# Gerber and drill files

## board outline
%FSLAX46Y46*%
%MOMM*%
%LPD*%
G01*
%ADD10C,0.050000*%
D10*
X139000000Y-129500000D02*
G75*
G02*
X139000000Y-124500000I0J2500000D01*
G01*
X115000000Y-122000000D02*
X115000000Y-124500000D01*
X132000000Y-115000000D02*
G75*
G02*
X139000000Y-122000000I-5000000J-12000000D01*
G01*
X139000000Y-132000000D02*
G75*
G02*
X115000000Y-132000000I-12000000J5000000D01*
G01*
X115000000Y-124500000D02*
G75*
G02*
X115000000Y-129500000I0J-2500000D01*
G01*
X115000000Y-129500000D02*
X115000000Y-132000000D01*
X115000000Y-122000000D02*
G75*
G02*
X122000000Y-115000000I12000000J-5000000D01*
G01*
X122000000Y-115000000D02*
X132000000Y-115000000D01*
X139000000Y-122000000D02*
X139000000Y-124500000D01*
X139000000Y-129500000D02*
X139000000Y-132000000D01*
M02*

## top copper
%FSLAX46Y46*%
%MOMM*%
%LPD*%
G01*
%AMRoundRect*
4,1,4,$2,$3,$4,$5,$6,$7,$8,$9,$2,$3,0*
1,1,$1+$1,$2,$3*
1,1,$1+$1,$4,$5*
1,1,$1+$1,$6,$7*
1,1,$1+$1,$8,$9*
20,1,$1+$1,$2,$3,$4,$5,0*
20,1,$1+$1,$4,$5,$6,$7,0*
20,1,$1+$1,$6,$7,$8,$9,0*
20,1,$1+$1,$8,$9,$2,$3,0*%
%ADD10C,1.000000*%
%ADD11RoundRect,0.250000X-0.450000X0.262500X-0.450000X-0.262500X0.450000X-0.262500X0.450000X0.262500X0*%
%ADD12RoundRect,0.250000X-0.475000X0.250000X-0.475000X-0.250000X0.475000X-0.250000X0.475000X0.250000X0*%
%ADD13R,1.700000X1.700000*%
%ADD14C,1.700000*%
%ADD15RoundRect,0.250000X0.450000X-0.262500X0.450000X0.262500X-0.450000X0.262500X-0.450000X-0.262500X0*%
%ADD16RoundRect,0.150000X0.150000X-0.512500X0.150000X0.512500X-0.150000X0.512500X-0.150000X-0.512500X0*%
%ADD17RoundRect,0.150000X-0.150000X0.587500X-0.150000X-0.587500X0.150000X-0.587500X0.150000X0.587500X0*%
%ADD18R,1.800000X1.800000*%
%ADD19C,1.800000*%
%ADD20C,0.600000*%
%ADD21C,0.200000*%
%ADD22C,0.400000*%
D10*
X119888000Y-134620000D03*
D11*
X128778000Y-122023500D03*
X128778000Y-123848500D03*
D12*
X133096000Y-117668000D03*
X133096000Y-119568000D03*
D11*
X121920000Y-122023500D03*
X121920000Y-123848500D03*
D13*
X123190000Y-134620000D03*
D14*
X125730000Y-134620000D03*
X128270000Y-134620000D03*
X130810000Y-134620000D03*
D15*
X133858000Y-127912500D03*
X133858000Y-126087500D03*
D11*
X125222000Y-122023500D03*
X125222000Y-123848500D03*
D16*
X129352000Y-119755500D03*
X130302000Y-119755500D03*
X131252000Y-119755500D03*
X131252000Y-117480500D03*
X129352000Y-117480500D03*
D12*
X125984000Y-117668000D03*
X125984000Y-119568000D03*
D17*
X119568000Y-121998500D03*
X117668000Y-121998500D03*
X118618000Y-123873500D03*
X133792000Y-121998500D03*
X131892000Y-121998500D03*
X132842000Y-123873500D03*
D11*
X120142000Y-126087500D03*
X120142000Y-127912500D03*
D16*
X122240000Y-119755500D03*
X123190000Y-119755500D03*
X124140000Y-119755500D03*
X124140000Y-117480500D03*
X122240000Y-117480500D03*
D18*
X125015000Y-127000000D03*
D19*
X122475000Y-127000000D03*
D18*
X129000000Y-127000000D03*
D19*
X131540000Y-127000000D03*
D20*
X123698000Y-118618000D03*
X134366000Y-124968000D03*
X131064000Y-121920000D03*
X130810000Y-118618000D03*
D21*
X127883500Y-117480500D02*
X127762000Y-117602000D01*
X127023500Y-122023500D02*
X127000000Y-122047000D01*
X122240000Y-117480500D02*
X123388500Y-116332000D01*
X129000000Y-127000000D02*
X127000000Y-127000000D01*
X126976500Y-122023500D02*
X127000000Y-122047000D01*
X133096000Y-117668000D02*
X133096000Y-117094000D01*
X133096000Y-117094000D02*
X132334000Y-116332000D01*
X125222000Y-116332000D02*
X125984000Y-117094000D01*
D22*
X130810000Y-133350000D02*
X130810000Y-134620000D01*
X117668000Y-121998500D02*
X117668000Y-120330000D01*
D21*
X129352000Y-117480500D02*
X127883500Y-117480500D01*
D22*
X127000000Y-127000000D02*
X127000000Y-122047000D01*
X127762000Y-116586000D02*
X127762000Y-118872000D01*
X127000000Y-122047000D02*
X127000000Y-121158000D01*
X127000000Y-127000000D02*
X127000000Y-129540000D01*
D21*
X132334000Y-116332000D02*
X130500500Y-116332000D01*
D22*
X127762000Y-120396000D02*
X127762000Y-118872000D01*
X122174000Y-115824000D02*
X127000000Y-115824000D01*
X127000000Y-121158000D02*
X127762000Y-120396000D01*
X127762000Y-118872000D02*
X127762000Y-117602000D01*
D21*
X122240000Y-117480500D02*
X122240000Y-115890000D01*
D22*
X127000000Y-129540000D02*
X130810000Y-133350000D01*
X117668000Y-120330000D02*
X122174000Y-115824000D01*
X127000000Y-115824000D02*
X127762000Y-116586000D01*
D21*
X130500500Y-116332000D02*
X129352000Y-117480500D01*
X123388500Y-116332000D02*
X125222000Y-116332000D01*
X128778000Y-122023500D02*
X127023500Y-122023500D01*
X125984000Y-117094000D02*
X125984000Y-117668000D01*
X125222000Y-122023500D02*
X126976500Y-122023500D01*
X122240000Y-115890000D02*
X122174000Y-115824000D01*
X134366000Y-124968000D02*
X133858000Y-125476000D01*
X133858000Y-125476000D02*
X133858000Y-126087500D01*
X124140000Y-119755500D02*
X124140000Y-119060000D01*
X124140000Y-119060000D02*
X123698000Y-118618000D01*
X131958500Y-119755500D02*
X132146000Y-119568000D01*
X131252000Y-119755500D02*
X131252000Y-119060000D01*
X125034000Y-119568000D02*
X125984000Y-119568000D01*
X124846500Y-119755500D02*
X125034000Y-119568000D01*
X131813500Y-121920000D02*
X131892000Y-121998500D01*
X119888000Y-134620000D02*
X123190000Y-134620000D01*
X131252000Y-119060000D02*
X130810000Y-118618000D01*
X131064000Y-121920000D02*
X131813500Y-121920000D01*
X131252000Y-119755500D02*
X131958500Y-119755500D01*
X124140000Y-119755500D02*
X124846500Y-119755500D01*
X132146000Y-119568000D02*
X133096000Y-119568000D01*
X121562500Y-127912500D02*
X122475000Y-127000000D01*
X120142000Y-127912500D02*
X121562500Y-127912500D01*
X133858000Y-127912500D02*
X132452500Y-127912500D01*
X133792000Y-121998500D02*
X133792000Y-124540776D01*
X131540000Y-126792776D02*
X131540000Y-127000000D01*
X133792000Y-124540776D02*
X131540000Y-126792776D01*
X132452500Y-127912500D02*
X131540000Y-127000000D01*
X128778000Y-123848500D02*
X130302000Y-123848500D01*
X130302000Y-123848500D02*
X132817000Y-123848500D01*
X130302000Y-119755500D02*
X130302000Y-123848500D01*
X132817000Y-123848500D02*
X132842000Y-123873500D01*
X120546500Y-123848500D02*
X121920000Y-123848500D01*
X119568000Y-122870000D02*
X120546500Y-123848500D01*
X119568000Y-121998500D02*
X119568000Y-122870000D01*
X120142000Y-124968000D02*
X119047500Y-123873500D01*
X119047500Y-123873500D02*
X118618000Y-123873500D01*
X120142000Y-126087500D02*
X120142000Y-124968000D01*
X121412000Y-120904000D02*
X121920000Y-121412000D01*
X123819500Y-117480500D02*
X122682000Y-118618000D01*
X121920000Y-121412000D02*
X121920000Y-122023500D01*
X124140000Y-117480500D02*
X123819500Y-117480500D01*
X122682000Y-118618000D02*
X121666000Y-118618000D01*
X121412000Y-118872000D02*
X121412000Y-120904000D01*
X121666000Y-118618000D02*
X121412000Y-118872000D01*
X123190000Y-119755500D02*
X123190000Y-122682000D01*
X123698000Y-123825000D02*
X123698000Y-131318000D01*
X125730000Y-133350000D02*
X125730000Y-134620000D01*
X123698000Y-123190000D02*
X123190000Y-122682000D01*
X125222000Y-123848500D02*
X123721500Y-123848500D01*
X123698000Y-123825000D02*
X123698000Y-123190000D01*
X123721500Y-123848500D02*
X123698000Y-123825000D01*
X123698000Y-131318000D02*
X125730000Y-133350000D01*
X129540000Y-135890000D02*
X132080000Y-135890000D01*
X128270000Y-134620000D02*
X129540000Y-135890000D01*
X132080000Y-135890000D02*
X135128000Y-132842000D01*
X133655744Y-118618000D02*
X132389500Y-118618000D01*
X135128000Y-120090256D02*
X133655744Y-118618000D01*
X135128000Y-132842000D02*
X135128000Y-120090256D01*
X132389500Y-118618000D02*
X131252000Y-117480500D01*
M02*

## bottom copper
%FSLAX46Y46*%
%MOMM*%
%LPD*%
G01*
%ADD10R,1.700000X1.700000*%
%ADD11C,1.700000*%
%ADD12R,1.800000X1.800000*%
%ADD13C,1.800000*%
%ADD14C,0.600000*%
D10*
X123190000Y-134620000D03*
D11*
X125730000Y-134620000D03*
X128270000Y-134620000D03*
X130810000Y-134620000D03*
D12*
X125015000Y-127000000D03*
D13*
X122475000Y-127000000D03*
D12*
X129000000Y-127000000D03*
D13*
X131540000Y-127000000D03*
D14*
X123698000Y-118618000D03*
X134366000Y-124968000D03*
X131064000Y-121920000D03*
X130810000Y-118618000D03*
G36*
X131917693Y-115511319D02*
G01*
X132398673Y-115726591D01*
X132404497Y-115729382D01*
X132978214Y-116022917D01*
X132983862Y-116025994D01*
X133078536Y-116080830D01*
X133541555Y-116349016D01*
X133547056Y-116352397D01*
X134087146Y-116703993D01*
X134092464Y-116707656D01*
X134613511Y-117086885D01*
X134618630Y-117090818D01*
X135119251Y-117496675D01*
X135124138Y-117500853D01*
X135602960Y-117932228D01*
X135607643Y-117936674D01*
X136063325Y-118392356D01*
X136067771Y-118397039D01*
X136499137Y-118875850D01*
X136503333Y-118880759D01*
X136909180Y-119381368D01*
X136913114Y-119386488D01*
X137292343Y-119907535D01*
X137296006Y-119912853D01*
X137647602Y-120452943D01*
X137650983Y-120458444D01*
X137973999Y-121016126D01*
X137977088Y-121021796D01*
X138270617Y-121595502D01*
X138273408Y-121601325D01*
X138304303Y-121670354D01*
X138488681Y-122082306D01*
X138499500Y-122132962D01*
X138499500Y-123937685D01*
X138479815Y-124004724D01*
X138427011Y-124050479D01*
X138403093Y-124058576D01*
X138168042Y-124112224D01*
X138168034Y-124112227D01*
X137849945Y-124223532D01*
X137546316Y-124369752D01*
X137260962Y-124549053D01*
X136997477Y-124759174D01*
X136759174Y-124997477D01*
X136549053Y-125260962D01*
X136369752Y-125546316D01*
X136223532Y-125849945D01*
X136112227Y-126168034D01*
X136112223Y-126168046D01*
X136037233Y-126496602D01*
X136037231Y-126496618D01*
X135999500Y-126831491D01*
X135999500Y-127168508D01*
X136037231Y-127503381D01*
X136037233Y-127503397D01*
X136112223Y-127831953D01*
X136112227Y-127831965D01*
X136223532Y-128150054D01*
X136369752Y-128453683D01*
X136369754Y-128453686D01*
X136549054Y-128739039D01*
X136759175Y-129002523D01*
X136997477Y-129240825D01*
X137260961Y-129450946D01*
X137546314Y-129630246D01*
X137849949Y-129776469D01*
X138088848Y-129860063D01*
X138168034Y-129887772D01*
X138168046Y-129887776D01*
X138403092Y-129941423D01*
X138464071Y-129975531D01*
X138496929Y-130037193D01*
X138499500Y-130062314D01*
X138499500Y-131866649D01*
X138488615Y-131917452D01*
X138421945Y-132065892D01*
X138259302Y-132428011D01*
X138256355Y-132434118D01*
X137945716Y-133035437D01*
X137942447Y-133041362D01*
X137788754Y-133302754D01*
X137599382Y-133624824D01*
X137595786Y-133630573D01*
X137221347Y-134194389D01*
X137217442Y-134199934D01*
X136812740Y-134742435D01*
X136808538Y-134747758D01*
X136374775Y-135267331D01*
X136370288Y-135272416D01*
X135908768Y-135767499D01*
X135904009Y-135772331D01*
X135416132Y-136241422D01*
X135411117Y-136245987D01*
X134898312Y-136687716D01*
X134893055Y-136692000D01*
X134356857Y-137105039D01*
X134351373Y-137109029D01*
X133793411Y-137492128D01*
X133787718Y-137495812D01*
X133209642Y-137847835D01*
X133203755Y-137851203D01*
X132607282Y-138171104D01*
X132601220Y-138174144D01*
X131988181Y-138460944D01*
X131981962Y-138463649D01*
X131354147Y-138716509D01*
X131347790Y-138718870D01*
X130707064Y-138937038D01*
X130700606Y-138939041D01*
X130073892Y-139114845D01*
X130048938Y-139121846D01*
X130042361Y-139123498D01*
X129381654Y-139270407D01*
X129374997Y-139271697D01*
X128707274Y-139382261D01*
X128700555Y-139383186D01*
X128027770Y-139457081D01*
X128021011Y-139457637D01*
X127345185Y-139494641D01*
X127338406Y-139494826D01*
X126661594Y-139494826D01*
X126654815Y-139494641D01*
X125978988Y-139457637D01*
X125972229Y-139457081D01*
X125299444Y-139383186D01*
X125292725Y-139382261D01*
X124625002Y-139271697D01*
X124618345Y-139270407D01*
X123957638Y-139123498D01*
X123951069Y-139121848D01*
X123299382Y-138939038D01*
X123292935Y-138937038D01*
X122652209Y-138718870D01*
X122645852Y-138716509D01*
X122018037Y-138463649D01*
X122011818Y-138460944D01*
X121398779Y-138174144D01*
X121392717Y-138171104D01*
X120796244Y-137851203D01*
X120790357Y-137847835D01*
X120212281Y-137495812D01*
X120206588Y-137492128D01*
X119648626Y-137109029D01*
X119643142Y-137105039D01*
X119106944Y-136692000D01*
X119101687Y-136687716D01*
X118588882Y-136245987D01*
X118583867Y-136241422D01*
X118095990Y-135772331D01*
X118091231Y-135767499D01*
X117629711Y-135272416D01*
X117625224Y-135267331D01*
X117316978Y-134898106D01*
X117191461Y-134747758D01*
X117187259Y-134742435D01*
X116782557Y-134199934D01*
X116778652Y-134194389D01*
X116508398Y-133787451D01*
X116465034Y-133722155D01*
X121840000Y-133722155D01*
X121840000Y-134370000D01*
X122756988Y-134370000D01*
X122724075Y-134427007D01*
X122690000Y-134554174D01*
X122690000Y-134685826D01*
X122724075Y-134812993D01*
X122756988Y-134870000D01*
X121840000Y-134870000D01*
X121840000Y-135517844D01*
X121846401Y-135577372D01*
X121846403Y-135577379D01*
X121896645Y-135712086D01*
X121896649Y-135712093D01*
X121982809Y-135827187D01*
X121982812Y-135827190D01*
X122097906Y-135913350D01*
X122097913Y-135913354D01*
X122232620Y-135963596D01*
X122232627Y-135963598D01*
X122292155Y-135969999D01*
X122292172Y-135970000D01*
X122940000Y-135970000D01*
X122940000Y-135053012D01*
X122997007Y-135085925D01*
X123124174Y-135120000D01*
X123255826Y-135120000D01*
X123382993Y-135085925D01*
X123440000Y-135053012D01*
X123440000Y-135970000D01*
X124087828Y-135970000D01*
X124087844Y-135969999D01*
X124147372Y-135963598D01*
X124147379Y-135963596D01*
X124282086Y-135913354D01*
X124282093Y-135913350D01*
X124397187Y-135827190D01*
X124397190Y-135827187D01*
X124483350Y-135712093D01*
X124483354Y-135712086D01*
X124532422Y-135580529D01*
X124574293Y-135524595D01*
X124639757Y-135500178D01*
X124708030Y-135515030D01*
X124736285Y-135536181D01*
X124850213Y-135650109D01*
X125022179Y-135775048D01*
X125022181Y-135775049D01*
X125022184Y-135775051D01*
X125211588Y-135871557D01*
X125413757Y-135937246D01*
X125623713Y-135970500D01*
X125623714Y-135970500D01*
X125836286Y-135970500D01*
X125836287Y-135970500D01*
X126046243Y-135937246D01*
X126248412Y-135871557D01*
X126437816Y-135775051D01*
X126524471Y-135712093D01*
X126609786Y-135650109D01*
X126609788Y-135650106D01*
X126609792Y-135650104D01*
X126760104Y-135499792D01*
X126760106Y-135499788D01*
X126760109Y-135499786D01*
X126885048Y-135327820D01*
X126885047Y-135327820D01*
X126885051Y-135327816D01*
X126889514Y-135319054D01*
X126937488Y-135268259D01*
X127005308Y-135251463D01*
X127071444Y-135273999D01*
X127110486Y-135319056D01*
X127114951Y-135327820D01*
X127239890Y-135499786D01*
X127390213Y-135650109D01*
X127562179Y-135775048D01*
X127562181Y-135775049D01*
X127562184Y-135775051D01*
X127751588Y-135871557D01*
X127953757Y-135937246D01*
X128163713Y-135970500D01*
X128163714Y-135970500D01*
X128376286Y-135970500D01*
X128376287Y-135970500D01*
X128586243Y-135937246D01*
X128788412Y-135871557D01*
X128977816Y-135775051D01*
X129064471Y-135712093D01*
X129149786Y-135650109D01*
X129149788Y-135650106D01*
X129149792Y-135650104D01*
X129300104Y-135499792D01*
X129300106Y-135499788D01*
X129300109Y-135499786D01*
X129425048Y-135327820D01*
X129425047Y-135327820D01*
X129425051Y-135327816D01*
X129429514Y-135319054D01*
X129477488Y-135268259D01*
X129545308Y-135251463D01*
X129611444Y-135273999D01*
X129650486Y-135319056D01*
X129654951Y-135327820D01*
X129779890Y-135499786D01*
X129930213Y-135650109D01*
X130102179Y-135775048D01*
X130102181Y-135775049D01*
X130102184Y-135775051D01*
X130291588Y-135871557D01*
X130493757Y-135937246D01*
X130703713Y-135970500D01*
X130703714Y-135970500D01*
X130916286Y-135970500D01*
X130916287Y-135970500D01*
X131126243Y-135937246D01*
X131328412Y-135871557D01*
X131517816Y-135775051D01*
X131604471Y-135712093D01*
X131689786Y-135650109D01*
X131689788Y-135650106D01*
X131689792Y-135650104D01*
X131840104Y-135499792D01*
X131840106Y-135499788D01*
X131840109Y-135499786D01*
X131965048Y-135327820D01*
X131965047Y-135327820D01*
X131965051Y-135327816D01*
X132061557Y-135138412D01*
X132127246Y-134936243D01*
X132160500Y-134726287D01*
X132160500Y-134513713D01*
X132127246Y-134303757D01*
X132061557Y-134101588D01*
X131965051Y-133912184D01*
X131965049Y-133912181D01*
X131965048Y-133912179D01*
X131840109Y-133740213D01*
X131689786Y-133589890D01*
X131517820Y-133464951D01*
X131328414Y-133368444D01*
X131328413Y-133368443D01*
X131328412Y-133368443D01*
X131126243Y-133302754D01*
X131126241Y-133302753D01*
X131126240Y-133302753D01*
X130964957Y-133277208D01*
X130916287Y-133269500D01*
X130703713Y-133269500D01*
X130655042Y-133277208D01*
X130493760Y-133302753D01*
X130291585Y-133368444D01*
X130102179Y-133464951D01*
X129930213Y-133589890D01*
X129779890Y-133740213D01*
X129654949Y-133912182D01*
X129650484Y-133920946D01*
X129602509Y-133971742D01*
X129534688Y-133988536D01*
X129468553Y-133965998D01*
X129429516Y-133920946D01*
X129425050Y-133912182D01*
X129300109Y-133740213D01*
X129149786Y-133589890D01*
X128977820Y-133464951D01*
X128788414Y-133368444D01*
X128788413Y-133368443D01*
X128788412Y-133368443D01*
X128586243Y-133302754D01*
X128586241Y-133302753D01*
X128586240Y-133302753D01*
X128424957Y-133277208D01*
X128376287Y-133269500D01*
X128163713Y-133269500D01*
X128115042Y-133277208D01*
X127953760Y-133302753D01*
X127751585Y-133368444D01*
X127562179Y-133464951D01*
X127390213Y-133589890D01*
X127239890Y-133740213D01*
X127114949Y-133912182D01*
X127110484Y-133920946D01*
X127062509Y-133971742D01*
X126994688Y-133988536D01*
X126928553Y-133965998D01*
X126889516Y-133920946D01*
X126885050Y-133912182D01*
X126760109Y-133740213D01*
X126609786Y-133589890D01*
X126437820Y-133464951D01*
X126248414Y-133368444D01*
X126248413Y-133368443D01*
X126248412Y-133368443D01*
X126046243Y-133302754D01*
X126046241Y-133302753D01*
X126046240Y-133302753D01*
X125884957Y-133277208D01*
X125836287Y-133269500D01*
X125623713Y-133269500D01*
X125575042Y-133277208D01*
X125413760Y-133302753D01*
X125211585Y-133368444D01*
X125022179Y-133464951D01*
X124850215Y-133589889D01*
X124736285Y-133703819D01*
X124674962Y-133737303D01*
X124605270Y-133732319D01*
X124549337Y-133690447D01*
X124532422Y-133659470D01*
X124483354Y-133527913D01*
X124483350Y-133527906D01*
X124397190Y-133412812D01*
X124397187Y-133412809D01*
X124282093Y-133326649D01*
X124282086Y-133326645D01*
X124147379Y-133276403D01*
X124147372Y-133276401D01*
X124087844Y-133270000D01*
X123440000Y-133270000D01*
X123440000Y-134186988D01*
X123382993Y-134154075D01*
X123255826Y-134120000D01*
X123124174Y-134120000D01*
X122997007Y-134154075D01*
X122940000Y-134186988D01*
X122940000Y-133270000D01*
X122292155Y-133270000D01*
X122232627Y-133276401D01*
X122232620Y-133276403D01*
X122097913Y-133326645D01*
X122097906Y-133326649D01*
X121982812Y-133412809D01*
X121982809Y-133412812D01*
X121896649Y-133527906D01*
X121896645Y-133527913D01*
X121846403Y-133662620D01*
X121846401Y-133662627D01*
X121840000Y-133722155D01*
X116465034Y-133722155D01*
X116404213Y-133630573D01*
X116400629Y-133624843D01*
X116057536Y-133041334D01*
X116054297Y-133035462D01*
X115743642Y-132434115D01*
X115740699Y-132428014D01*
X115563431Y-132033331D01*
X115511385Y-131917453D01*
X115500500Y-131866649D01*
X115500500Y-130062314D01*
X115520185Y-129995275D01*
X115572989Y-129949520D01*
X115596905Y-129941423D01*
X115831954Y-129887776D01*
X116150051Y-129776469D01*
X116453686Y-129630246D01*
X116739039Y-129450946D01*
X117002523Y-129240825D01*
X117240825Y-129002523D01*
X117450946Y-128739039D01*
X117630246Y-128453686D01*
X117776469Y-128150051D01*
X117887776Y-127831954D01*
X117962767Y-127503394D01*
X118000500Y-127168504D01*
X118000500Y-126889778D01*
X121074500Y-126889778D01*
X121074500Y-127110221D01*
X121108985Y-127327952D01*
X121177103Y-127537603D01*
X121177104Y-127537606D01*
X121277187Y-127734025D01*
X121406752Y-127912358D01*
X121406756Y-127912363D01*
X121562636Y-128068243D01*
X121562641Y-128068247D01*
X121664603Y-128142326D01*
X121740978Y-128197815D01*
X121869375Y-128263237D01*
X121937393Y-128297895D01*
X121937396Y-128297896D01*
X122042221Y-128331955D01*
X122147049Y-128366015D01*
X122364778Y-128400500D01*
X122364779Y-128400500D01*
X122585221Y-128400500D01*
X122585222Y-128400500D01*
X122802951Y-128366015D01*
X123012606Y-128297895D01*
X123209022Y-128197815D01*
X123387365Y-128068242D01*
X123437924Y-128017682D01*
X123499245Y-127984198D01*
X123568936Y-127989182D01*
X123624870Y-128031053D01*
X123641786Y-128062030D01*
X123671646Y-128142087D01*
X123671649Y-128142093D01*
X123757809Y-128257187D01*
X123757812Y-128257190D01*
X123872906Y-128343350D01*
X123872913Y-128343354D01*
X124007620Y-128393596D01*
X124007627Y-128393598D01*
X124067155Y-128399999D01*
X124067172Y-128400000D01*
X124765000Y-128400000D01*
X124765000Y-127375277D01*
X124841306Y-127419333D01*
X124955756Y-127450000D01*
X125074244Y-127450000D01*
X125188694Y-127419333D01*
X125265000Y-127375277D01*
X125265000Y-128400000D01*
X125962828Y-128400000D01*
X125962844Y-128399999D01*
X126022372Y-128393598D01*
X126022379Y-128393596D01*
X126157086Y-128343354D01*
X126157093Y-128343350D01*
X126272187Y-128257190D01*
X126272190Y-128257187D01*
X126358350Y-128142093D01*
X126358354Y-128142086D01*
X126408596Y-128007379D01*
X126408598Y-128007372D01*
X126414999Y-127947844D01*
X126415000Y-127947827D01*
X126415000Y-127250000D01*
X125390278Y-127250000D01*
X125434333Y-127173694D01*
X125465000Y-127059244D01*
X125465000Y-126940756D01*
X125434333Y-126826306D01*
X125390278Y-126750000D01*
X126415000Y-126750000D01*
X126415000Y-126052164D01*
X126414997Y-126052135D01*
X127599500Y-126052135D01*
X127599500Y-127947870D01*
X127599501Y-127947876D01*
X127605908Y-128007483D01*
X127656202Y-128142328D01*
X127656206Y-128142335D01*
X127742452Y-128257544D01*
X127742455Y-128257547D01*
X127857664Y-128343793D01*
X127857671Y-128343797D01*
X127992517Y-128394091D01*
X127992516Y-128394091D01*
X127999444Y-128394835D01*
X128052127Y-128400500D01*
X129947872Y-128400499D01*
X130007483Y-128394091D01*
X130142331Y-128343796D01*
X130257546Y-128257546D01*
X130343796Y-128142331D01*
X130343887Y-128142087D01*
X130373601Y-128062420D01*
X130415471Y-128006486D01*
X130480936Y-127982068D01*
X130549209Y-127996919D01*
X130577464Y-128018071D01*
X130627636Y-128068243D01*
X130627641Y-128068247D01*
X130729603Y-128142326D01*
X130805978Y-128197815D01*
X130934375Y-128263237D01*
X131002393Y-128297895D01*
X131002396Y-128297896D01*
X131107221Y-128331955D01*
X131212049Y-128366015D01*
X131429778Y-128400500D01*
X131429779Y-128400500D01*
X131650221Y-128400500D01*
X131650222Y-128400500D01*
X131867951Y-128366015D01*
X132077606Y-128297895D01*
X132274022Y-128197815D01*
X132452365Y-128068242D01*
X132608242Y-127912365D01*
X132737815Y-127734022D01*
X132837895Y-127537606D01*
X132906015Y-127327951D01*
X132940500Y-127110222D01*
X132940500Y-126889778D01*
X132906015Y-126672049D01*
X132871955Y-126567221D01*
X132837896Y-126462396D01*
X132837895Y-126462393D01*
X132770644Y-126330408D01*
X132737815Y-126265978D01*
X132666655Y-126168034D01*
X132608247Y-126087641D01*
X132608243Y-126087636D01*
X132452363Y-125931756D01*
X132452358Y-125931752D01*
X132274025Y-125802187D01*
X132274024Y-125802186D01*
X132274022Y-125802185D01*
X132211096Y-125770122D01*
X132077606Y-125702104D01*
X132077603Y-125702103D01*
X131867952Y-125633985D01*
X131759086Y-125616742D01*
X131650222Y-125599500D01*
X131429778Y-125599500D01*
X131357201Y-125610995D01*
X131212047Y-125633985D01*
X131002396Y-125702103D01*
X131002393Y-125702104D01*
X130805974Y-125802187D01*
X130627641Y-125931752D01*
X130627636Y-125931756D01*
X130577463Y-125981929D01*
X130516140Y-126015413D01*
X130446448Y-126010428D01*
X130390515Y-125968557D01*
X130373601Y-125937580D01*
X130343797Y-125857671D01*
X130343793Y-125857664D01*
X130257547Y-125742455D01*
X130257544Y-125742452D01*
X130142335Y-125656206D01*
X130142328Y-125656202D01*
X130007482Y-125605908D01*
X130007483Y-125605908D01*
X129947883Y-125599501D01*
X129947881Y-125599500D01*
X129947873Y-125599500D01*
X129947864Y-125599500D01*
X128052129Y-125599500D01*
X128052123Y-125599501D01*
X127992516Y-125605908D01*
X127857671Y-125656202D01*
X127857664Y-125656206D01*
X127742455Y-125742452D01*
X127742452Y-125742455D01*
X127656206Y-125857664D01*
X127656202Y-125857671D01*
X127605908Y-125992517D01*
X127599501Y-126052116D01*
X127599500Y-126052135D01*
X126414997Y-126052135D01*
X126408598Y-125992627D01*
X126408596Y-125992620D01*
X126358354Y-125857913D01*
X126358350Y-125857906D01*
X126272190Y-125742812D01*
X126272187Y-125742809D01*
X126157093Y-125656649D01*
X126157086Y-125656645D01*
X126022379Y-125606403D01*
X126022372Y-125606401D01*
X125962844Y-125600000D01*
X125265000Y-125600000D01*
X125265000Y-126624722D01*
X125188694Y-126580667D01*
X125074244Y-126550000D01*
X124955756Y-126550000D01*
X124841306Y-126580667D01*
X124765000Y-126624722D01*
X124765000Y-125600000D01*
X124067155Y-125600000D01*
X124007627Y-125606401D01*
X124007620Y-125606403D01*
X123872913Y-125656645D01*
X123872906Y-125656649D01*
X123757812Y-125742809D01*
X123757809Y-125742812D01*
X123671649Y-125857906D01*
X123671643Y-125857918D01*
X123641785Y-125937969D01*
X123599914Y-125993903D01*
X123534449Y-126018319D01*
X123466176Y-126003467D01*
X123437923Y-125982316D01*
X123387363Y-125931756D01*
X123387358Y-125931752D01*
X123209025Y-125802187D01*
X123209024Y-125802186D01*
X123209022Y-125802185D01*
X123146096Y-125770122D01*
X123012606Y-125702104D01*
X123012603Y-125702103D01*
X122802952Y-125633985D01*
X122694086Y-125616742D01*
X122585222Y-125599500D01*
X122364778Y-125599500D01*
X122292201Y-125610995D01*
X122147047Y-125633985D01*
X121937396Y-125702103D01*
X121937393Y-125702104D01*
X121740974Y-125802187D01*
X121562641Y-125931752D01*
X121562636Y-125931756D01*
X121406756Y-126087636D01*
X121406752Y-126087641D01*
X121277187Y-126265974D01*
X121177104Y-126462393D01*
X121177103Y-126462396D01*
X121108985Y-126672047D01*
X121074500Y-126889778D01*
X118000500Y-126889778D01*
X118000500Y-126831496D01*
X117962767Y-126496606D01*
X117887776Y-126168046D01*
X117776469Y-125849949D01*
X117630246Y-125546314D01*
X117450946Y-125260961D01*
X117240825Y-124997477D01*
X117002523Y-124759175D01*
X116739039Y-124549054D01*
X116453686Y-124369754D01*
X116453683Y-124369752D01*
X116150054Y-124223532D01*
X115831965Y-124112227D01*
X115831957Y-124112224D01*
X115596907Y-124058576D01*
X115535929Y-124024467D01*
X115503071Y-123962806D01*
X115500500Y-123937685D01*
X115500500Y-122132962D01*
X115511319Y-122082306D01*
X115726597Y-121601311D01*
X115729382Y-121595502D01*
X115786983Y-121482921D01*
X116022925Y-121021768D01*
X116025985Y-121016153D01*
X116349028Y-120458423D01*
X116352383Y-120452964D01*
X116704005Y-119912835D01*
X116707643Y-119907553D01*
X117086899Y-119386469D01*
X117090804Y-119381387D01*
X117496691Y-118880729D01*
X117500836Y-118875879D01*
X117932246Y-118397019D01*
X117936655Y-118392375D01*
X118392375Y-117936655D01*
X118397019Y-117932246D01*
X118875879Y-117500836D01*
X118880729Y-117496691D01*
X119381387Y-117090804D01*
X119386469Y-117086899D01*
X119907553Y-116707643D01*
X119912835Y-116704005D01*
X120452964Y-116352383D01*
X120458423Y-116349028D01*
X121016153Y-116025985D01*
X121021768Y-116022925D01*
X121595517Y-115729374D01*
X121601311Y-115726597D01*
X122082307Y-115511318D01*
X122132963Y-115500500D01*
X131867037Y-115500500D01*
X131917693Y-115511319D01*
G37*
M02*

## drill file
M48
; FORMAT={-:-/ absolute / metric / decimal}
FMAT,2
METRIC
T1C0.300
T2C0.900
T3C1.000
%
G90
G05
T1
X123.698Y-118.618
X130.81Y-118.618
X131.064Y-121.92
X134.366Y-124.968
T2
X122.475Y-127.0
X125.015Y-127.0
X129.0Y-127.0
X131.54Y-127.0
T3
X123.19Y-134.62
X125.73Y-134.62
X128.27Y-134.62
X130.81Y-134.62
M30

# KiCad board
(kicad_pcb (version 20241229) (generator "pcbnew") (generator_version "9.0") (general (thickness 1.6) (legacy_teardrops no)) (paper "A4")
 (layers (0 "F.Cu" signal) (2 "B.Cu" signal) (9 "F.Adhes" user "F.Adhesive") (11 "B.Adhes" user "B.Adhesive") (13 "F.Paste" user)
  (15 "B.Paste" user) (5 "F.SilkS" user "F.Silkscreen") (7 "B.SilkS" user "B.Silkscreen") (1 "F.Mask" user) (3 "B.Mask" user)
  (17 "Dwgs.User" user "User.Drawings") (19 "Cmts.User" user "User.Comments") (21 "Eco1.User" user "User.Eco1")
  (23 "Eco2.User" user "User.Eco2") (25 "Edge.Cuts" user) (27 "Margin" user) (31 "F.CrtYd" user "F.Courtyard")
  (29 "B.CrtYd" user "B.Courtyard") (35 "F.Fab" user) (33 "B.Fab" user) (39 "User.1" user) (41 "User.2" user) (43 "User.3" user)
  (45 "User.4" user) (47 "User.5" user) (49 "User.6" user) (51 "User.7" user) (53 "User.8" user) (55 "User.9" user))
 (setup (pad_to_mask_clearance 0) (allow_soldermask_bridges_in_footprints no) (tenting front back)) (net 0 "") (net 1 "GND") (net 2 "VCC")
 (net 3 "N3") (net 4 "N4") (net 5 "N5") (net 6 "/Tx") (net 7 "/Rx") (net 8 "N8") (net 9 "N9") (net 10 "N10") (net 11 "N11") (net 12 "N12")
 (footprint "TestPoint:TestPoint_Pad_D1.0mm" (layer "F.Cu") (at 119.888 134.62)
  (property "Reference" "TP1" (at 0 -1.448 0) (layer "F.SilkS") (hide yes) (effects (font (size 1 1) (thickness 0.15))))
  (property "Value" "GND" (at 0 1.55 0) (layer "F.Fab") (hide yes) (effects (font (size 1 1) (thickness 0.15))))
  (pad "1" smd circle (at 0 0) (size 1 1) (layers "F.Cu" "F.Mask") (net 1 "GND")))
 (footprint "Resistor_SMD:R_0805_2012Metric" (layer "F.Cu") (at 128.778 122.936 -90)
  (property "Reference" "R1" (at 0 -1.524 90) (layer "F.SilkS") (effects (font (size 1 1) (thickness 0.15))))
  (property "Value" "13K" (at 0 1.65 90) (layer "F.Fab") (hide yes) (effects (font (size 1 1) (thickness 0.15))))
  (pad "1" smd roundrect (at -0.9125 0 270) (size 1.025 1.4) (layers "F.Cu" "F.Mask" "F.Paste") (roundrect_rratio 0.243902) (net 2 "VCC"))
  (pad "2" smd roundrect (at 0.9125 0 270) (size 1.025 1.4) (layers "F.Cu" "F.Mask" "F.Paste") (roundrect_rratio 0.243902) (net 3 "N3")))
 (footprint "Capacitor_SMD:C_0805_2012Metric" (layer "F.Cu") (at 133.096 118.618 -90)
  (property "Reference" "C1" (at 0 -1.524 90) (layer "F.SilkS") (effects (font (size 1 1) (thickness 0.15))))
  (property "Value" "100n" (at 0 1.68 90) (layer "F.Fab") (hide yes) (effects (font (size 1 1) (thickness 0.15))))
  (pad "1" smd roundrect (at -0.95 0 270) (size 1 1.45) (layers "F.Cu" "F.Mask" "F.Paste") (roundrect_rratio 0.25) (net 2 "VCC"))
  (pad "2" smd roundrect (at 0.95 0 270) (size 1 1.45) (layers "F.Cu" "F.Mask" "F.Paste") (roundrect_rratio 0.25) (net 1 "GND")))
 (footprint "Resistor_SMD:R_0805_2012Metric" (layer "F.Cu") (at 121.92 122.936 -90)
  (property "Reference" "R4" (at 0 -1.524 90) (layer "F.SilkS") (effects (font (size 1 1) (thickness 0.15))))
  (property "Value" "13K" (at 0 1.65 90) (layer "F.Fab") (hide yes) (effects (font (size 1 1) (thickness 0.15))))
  (pad "1" smd roundrect (at -0.9125 0 270) (size 1.025 1.4) (layers "F.Cu" "F.Mask" "F.Paste") (roundrect_rratio 0.243902) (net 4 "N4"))
  (pad "2" smd roundrect (at 0.9125 0 270) (size 1.025 1.4) (layers "F.Cu" "F.Mask" "F.Paste") (roundrect_rratio 0.243902) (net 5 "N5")))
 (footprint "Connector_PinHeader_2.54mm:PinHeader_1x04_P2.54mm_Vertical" (layer "F.Cu") (at 123.19 134.62 90)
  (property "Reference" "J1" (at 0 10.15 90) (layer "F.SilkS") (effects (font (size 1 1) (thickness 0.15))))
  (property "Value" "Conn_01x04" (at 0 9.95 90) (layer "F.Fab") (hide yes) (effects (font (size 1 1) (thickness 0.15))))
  (pad "1" thru_hole rect (at 0 0 90) (size 1.7 1.7) (drill 1) (layers "*.Cu" "*.Mask") (remove_unused_layers no) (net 1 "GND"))
  (pad "2" thru_hole circle (at 0 2.54 90) (size 1.7 1.7) (drill 1) (layers "*.Cu" "*.Mask") (remove_unused_layers no) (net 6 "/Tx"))
  (pad "3" thru_hole circle (at 0 5.08 90) (size 1.7 1.7) (drill 1) (layers "*.Cu" "*.Mask") (remove_unused_layers no) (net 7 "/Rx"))
  (pad "4" thru_hole circle (at 0 7.62 90) (size 1.7 1.7) (drill 1) (layers "*.Cu" "*.Mask") (remove_unused_layers no) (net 2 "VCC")))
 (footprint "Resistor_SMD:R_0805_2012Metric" (layer "F.Cu") (at 133.858 127 90)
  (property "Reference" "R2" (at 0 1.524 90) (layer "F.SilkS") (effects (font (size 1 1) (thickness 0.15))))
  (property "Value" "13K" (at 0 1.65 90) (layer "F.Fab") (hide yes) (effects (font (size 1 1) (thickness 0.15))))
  (pad "1" smd roundrect (at -0.9125 0 90) (size 1.025 1.4) (layers "F.Cu" "F.Mask" "F.Paste") (roundrect_rratio 0.243902) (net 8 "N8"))
  (pad "2" smd roundrect (at 0.9125 0 90) (size 1.025 1.4) (layers "F.Cu" "F.Mask" "F.Paste") (roundrect_rratio 0.243902) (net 1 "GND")))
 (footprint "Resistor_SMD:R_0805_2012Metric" (layer "F.Cu") (at 125.222 122.936 -90)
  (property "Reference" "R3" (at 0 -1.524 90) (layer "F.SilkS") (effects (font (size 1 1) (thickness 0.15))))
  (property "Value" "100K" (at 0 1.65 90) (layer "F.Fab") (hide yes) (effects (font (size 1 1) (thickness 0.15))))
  (pad "1" smd roundrect (at -0.9125 0 270) (size 1.025 1.4) (layers "F.Cu" "F.Mask" "F.Paste") (roundrect_rratio 0.243902) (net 2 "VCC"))
  (pad "2" smd roundrect (at 0.9125 0 270) (size 1.025 1.4) (layers "F.Cu" "F.Mask" "F.Paste") (roundrect_rratio 0.243902) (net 6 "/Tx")))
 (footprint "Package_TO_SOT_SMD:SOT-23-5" (layer "F.Cu") (at 130.302 118.618 90)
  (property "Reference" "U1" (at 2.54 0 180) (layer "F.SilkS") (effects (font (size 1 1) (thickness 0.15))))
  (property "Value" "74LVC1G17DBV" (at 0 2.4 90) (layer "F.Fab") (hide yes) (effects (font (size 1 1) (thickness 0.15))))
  (pad "1" smd roundrect (at -1.1375 -0.95 90) (size 1.325 0.6) (layers "F.Cu" "F.Mask" "F.Paste") (roundrect_rratio 0.25) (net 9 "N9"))
  (pad "2" smd roundrect (at -1.1375 0 90) (size 1.325 0.6) (layers "F.Cu" "F.Mask" "F.Paste") (roundrect_rratio 0.25) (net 3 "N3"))
  (pad "3" smd roundrect (at -1.1375 0.95 90) (size 1.325 0.6) (layers "F.Cu" "F.Mask" "F.Paste") (roundrect_rratio 0.25) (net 1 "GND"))
  (pad "4" smd roundrect (at 1.1375 0.95 90) (size 1.325 0.6) (layers "F.Cu" "F.Mask" "F.Paste") (roundrect_rratio 0.25) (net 7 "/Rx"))
  (pad "5" smd roundrect (at 1.1375 -0.95 90) (size 1.325 0.6) (layers "F.Cu" "F.Mask" "F.Paste") (roundrect_rratio 0.25) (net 2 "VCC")))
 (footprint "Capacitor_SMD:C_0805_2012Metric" (layer "F.Cu") (at 125.984 118.618 -90)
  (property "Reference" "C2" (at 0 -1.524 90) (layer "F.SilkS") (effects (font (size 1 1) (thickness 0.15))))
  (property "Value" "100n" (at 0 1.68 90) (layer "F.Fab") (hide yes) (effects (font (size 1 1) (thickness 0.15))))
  (pad "1" smd roundrect (at -0.95 0 270) (size 1 1.45) (layers "F.Cu" "F.Mask" "F.Paste") (roundrect_rratio 0.25) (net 2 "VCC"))
  (pad "2" smd roundrect (at 0.95 0 270) (size 1 1.45) (layers "F.Cu" "F.Mask" "F.Paste") (roundrect_rratio 0.25) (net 1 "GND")))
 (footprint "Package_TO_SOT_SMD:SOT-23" (layer "F.Cu") (at 118.618 122.936 -90)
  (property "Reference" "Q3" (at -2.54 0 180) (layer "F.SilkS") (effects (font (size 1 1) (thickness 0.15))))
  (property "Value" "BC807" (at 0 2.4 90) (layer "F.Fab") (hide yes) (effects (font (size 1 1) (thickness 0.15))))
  (pad "1" smd roundrect (at -0.9375 -0.95 270) (size 1.475 0.6) (layers "F.Cu" "F.Mask" "F.Paste") (roundrect_rratio 0.25) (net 5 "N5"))
  (pad "2" smd roundrect (at -0.9375 0.95 270) (size 1.475 0.6) (layers "F.Cu" "F.Mask" "F.Paste") (roundrect_rratio 0.25) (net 2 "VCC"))
  (pad "3" smd roundrect (at 0.9375 0 270) (size 1.475 0.6) (layers "F.Cu" "F.Mask" "F.Paste") (roundrect_rratio 0.25) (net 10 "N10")))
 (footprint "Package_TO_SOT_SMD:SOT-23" (layer "F.Cu") (at 132.842 122.936 -90)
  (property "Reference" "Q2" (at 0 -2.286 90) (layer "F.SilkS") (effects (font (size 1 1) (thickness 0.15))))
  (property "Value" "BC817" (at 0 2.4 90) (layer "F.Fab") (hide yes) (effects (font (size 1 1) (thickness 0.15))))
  (pad "1" smd roundrect (at -0.9375 -0.95 270) (size 1.475 0.6) (layers "F.Cu" "F.Mask" "F.Paste") (roundrect_rratio 0.25) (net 8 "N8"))
  (pad "2" smd roundrect (at -0.9375 0.95 270) (size 1.475 0.6) (layers "F.Cu" "F.Mask" "F.Paste") (roundrect_rratio 0.25) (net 1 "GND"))
  (pad "3" smd roundrect (at 0.9375 0 270) (size 1.475 0.6) (layers "F.Cu" "F.Mask" "F.Paste") (roundrect_rratio 0.25) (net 3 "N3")))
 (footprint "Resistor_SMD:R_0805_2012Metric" (layer "F.Cu") (at 120.142 127 -90)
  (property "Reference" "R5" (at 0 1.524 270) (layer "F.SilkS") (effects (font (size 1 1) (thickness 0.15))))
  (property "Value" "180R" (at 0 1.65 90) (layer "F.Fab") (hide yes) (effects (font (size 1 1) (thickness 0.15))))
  (pad "1" smd roundrect (at -0.9125 0 270) (size 1.025 1.4) (layers "F.Cu" "F.Mask" "F.Paste") (roundrect_rratio 0.243902) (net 10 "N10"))
  (pad "2" smd roundrect (at 0.9125 0 270) (size 1.025 1.4) (layers "F.Cu" "F.Mask" "F.Paste") (roundrect_rratio 0.243902) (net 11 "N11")))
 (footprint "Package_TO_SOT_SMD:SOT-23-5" (layer "F.Cu") (at 123.19 118.618 90)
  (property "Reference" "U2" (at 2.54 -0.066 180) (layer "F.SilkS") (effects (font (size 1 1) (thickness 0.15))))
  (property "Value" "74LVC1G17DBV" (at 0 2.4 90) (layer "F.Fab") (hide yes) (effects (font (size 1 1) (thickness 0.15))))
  (pad "1" smd roundrect (at -1.1375 -0.95 90) (size 1.325 0.6) (layers "F.Cu" "F.Mask" "F.Paste") (roundrect_rratio 0.25) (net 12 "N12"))
  (pad "2" smd roundrect (at -1.1375 0 90) (size 1.325 0.6) (layers "F.Cu" "F.Mask" "F.Paste") (roundrect_rratio 0.25) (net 6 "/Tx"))
  (pad "3" smd roundrect (at -1.1375 0.95 90) (size 1.325 0.6) (layers "F.Cu" "F.Mask" "F.Paste") (roundrect_rratio 0.25) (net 1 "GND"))
  (pad "4" smd roundrect (at 1.1375 0.95 90) (size 1.325 0.6) (layers "F.Cu" "F.Mask" "F.Paste") (roundrect_rratio 0.25) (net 4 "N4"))
  (pad "5" smd roundrect (at 1.1375 -0.95 90) (size 1.325 0.6) (layers "F.Cu" "F.Mask" "F.Paste") (roundrect_rratio 0.25) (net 2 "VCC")))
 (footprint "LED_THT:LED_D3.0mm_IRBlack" (layer "B.Cu") (at 125.015 127 180)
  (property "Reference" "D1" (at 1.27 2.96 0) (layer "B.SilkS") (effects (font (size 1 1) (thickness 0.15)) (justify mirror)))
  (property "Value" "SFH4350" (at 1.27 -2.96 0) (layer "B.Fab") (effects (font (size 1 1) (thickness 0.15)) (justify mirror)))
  (pad "1" thru_hole rect (at 0 0 180) (size 1.8 1.8) (drill 0.9) (layers "*.Cu" "*.Mask") (remove_unused_layers no) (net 1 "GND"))
  (pad "2" thru_hole circle (at 2.54 0 180) (size 1.8 1.8) (drill 0.9) (layers "*.Cu" "*.Mask") (remove_unused_layers no) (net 11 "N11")))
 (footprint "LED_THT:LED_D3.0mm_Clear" (layer "B.Cu") (at 129 127)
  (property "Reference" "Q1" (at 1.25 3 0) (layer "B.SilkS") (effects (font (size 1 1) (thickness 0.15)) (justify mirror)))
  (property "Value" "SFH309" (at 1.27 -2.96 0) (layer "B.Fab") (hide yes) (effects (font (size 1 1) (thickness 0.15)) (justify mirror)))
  (pad "1" thru_hole rect (at 0 0) (size 1.8 1.8) (drill 0.9) (layers "*.Cu" "*.Mask") (remove_unused_layers no) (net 2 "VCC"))
  (pad "2" thru_hole circle (at 2.54 0) (size 1.8 1.8) (drill 0.9) (layers "*.Cu" "*.Mask") (remove_unused_layers no) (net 8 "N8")))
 (gr_arc (start 139 129.5) (mid 136.5 127) (end 139 124.5) (stroke (width 0.05) (type default)) (layer "Edge.Cuts"))
 (gr_line (start 115 122) (end 115 124.5) (stroke (width 0.05) (type default)) (layer "Edge.Cuts"))
 (gr_arc (start 132 115) (mid 136.192388 117.807612) (end 139 122) (stroke (width 0.05) (type default)) (layer "Edge.Cuts"))
 (gr_arc (start 139 132) (mid 127 140) (end 115 132) (stroke (width 0.05) (type default)) (layer "Edge.Cuts"))
 (gr_arc (start 115 124.5) (mid 117.5 127) (end 115 129.5) (stroke (width 0.05) (type default)) (layer "Edge.Cuts"))
 (gr_line (start 115 129.5) (end 115 132) (stroke (width 0.05) (type default)) (layer "Edge.Cuts"))
 (gr_arc (start 115 122) (mid 117.807612 117.807612) (end 122 115) (stroke (width 0.05) (type default)) (layer "Edge.Cuts"))
 (gr_line (start 122 115) (end 132 115) (stroke (width 0.05) (type default)) (layer "Edge.Cuts"))
 (gr_line (start 139 122) (end 139 124.5) (stroke (width 0.05) (type default)) (layer "Edge.Cuts"))
 (gr_line (start 139 129.5) (end 139 132) (stroke (width 0.05) (type default)) (layer "Edge.Cuts"))
 (segment (start 127.8835 117.4805) (end 127.762 117.602) (width 0.2) (layer "F.Cu") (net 2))
 (segment (start 127.0235 122.0235) (end 127 122.047) (width 0.2) (layer "F.Cu") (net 2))
 (segment (start 122.24 117.4805) (end 123.3885 116.332) (width 0.2) (layer "F.Cu") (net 2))
 (segment (start 129 127) (end 127 127) (width 0.2) (layer "F.Cu") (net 2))
 (segment (start 126.9765 122.0235) (end 127 122.047) (width 0.2) (layer "F.Cu") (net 2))
 (segment (start 133.096 117.668) (end 133.096 117.094) (width 0.2) (layer "F.Cu") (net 2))
 (segment (start 133.096 117.094) (end 132.334 116.332) (width 0.2) (layer "F.Cu") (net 2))
 (segment (start 125.222 116.332) (end 125.984 117.094) (width 0.2) (layer "F.Cu") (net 2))
 (segment (start 130.81 133.35) (end 130.81 134.62) (width 0.4) (layer "F.Cu") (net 2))
 (segment (start 117.668 121.9985) (end 117.668 120.33) (width 0.4) (layer "F.Cu") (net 2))
 (segment (start 129.352 117.4805) (end 127.8835 117.4805) (width 0.2) (layer "F.Cu") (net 2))
 (segment (start 127 127) (end 127 122.047) (width 0.4) (layer "F.Cu") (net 2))
 (segment (start 127.762 116.586) (end 127.762 118.872) (width 0.4) (layer "F.Cu") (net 2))
 (segment (start 127 122.047) (end 127 121.158) (width 0.4) (layer "F.Cu") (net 2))
 (segment (start 127 127) (end 127 129.54) (width 0.4) (layer "F.Cu") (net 2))
 (segment (start 132.334 116.332) (end 130.5005 116.332) (width 0.2) (layer "F.Cu") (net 2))
 (segment (start 127.762 120.396) (end 127.762 118.872) (width 0.4) (layer "F.Cu") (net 2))
 (segment (start 122.174 115.824) (end 127 115.824) (width 0.4) (layer "F.Cu") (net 2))
 (segment (start 127 121.158) (end 127.762 120.396) (width 0.4) (layer "F.Cu") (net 2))
 (segment (start 127.762 118.872) (end 127.762 117.602) (width 0.4) (layer "F.Cu") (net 2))
 (segment (start 122.24 117.4805) (end 122.24 115.89) (width 0.2) (layer "F.Cu") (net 2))
 (segment (start 127 129.54) (end 130.81 133.35) (width 0.4) (layer "F.Cu") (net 2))
 (segment (start 117.668 120.33) (end 122.174 115.824) (width 0.4) (layer "F.Cu") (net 2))
 (segment (start 127 115.824) (end 127.762 116.586) (width 0.4) (layer "F.Cu") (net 2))
 (segment (start 130.5005 116.332) (end 129.352 117.4805) (width 0.2) (layer "F.Cu") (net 2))
 (segment (start 123.3885 116.332) (end 125.222 116.332) (width 0.2) (layer "F.Cu") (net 2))
 (segment (start 128.778 122.0235) (end 127.0235 122.0235) (width 0.2) (layer "F.Cu") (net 2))
 (segment (start 125.984 117.094) (end 125.984 117.668) (width 0.2) (layer "F.Cu") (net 2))
 (segment (start 125.222 122.0235) (end 126.9765 122.0235) (width 0.2) (layer "F.Cu") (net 2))
 (segment (start 122.24 115.89) (end 122.174 115.824) (width 0.2) (layer "F.Cu") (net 2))
 (segment (start 134.366 124.968) (end 133.858 125.476) (width 0.2) (layer "F.Cu") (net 1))
 (segment (start 133.858 125.476) (end 133.858 126.0875) (width 0.2) (layer "F.Cu") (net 1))
 (segment (start 124.14 119.7555) (end 124.14 119.06) (width 0.2) (layer "F.Cu") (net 1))
 (segment (start 124.14 119.06) (end 123.698 118.618) (width 0.2) (layer "F.Cu") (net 1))
 (segment (start 131.9585 119.7555) (end 132.146 119.568) (width 0.2) (layer "F.Cu") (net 1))
 (segment (start 131.252 119.7555) (end 131.252 119.06) (width 0.2) (layer "F.Cu") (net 1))
 (segment (start 125.034 119.568) (end 125.984 119.568) (width 0.2) (layer "F.Cu") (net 1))
 (segment (start 124.8465 119.7555) (end 125.034 119.568) (width 0.2) (layer "F.Cu") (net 1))
 (segment (start 131.8135 121.92) (end 131.892 121.9985) (width 0.2) (layer "F.Cu") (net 1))
 (segment (start 119.888 134.62) (end 123.19 134.62) (width 0.2) (layer "F.Cu") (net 1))
 (segment (start 131.252 119.06) (end 130.81 118.618) (width 0.2) (layer "F.Cu") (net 1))
 (segment (start 131.064 121.92) (end 131.8135 121.92) (width 0.2) (layer "F.Cu") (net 1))
 (segment (start 131.252 119.7555) (end 131.9585 119.7555) (width 0.2) (layer "F.Cu") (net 1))
 (segment (start 124.14 119.7555) (end 124.8465 119.7555) (width 0.2) (layer "F.Cu") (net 1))
 (segment (start 132.146 119.568) (end 133.096 119.568) (width 0.2) (layer "F.Cu") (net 1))
 (via (at 123.698 118.618) (size 0.6) (drill 0.3) (layers "F.Cu" "B.Cu") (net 1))
 (via (at 134.366 124.968) (size 0.6) (drill 0.3) (layers "F.Cu" "B.Cu") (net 1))
 (via (at 131.064 121.92) (size 0.6) (drill 0.3) (layers "F.Cu" "B.Cu") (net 1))
 (via (at 130.81 118.618) (size 0.6) (drill 0.3) (layers "F.Cu" "B.Cu") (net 1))
 (segment (start 121.5625 127.9125) (end 122.475 127) (width 0.2) (layer "F.Cu") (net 11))
 (segment (start 120.142 127.9125) (end 121.5625 127.9125) (width 0.2) (layer "F.Cu") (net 11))
 (segment (start 133.858 127.9125) (end 132.4525 127.9125) (width 0.2) (layer "F.Cu") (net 8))
 (segment (start 133.792 121.9985) (end 133.792 124.540776) (width 0.2) (layer "F.Cu") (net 8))
 (segment (start 131.54 126.792776) (end 131.54 127) (width 0.2) (layer "F.Cu") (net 8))
 (segment (start 133.792 124.540776) (end 131.54 126.792776) (width 0.2) (layer "F.Cu") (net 8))
 (segment (start 132.4525 127.9125) (end 131.54 127) (width 0.2) (layer "F.Cu") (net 8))
 (segment (start 128.778 123.8485) (end 130.302 123.8485) (width 0.2) (layer "F.Cu") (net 3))
 (segment (start 130.302 123.8485) (end 132.817 123.8485) (width 0.2) (layer "F.Cu") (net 3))
 (segment (start 130.302 119.7555) (end 130.302 123.8485) (width 0.2) (layer "F.Cu") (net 3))
 (segment (start 132.817 123.8485) (end 132.842 123.8735) (width 0.2) (layer "F.Cu") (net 3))
 (segment (start 120.5465 123.8485) (end 121.92 123.8485) (width 0.2) (layer "F.Cu") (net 5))
 (segment (start 119.568 122.87) (end 120.5465 123.8485) (width 0.2) (layer "F.Cu") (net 5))
 (segment (start 119.568 121.9985) (end 119.568 122.87) (width 0.2) (layer "F.Cu") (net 5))
 (segment (start 120.142 124.968) (end 119.0475 123.8735) (width 0.2) (layer "F.Cu") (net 10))
 (segment (start 119.0475 123.8735) (end 118.618 123.8735) (width 0.2) (layer "F.Cu") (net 10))
 (segment (start 120.142 126.0875) (end 120.142 124.968) (width 0.2) (layer "F.Cu") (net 10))
 (segment (start 121.412 120.904) (end 121.92 121.412) (width 0.2) (layer "F.Cu") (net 4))
 (segment (start 123.8195 117.4805) (end 122.682 118.618) (width 0.2) (layer "F.Cu") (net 4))
 (segment (start 121.92 121.412) (end 121.92 122.0235) (width 0.2) (layer "F.Cu") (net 4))
 (segment (start 124.14 117.4805) (end 123.8195 117.4805) (width 0.2) (layer "F.Cu") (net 4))
 (segment (start 122.682 118.618) (end 121.666 118.618) (width 0.2) (layer "F.Cu") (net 4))
 (segment (start 121.412 118.872) (end 121.412 120.904) (width 0.2) (layer "F.Cu") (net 4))
 (segment (start 121.666 118.618) (end 121.412 118.872) (width 0.2) (layer "F.Cu") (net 4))
 (segment (start 123.19 119.7555) (end 123.19 122.682) (width 0.2) (layer "F.Cu") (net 6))
 (segment (start 123.698 123.825) (end 123.698 131.318) (width 0.2) (layer "F.Cu") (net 6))
 (segment (start 125.73 133.35) (end 125.73 134.62) (width 0.2) (layer "F.Cu") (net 6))
 (segment (start 123.698 123.19) (end 123.19 122.682) (width 0.2) (layer "F.Cu") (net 6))
 (segment (start 125.222 123.8485) (end 123.7215 123.8485) (width 0.2) (layer "F.Cu") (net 6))
 (segment (start 123.698 123.825) (end 123.698 123.19) (width 0.2) (layer "F.Cu") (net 6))
 (segment (start 123.7215 123.8485) (end 123.698 123.825) (width 0.2) (layer "F.Cu") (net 6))
 (segment (start 123.698 131.318) (end 125.73 133.35) (width 0.2) (layer "F.Cu") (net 6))
 (segment (start 129.54 135.89) (end 132.08 135.89) (width 0.2) (layer "F.Cu") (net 7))
 (segment (start 128.27 134.62) (end 129.54 135.89) (width 0.2) (layer "F.Cu") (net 7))
 (segment (start 132.08 135.89) (end 135.128 132.842) (width 0.2) (layer "F.Cu") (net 7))
 (segment (start 133.655744 118.618) (end 132.3895 118.618) (width 0.2) (layer "F.Cu") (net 7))
 (segment (start 135.128 120.090256) (end 133.655744 118.618) (width 0.2) (layer "F.Cu") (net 7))
 (segment (start 135.128 132.842) (end 135.128 120.090256) (width 0.2) (layer "F.Cu") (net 7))
 (segment (start 132.3895 118.618) (end 131.252 117.4805) (width 0.2) (layer "F.Cu") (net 7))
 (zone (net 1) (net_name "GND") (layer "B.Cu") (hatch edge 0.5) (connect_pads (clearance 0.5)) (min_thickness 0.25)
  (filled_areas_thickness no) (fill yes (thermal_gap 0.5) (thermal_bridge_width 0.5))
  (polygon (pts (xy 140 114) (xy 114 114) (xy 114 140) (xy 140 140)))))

